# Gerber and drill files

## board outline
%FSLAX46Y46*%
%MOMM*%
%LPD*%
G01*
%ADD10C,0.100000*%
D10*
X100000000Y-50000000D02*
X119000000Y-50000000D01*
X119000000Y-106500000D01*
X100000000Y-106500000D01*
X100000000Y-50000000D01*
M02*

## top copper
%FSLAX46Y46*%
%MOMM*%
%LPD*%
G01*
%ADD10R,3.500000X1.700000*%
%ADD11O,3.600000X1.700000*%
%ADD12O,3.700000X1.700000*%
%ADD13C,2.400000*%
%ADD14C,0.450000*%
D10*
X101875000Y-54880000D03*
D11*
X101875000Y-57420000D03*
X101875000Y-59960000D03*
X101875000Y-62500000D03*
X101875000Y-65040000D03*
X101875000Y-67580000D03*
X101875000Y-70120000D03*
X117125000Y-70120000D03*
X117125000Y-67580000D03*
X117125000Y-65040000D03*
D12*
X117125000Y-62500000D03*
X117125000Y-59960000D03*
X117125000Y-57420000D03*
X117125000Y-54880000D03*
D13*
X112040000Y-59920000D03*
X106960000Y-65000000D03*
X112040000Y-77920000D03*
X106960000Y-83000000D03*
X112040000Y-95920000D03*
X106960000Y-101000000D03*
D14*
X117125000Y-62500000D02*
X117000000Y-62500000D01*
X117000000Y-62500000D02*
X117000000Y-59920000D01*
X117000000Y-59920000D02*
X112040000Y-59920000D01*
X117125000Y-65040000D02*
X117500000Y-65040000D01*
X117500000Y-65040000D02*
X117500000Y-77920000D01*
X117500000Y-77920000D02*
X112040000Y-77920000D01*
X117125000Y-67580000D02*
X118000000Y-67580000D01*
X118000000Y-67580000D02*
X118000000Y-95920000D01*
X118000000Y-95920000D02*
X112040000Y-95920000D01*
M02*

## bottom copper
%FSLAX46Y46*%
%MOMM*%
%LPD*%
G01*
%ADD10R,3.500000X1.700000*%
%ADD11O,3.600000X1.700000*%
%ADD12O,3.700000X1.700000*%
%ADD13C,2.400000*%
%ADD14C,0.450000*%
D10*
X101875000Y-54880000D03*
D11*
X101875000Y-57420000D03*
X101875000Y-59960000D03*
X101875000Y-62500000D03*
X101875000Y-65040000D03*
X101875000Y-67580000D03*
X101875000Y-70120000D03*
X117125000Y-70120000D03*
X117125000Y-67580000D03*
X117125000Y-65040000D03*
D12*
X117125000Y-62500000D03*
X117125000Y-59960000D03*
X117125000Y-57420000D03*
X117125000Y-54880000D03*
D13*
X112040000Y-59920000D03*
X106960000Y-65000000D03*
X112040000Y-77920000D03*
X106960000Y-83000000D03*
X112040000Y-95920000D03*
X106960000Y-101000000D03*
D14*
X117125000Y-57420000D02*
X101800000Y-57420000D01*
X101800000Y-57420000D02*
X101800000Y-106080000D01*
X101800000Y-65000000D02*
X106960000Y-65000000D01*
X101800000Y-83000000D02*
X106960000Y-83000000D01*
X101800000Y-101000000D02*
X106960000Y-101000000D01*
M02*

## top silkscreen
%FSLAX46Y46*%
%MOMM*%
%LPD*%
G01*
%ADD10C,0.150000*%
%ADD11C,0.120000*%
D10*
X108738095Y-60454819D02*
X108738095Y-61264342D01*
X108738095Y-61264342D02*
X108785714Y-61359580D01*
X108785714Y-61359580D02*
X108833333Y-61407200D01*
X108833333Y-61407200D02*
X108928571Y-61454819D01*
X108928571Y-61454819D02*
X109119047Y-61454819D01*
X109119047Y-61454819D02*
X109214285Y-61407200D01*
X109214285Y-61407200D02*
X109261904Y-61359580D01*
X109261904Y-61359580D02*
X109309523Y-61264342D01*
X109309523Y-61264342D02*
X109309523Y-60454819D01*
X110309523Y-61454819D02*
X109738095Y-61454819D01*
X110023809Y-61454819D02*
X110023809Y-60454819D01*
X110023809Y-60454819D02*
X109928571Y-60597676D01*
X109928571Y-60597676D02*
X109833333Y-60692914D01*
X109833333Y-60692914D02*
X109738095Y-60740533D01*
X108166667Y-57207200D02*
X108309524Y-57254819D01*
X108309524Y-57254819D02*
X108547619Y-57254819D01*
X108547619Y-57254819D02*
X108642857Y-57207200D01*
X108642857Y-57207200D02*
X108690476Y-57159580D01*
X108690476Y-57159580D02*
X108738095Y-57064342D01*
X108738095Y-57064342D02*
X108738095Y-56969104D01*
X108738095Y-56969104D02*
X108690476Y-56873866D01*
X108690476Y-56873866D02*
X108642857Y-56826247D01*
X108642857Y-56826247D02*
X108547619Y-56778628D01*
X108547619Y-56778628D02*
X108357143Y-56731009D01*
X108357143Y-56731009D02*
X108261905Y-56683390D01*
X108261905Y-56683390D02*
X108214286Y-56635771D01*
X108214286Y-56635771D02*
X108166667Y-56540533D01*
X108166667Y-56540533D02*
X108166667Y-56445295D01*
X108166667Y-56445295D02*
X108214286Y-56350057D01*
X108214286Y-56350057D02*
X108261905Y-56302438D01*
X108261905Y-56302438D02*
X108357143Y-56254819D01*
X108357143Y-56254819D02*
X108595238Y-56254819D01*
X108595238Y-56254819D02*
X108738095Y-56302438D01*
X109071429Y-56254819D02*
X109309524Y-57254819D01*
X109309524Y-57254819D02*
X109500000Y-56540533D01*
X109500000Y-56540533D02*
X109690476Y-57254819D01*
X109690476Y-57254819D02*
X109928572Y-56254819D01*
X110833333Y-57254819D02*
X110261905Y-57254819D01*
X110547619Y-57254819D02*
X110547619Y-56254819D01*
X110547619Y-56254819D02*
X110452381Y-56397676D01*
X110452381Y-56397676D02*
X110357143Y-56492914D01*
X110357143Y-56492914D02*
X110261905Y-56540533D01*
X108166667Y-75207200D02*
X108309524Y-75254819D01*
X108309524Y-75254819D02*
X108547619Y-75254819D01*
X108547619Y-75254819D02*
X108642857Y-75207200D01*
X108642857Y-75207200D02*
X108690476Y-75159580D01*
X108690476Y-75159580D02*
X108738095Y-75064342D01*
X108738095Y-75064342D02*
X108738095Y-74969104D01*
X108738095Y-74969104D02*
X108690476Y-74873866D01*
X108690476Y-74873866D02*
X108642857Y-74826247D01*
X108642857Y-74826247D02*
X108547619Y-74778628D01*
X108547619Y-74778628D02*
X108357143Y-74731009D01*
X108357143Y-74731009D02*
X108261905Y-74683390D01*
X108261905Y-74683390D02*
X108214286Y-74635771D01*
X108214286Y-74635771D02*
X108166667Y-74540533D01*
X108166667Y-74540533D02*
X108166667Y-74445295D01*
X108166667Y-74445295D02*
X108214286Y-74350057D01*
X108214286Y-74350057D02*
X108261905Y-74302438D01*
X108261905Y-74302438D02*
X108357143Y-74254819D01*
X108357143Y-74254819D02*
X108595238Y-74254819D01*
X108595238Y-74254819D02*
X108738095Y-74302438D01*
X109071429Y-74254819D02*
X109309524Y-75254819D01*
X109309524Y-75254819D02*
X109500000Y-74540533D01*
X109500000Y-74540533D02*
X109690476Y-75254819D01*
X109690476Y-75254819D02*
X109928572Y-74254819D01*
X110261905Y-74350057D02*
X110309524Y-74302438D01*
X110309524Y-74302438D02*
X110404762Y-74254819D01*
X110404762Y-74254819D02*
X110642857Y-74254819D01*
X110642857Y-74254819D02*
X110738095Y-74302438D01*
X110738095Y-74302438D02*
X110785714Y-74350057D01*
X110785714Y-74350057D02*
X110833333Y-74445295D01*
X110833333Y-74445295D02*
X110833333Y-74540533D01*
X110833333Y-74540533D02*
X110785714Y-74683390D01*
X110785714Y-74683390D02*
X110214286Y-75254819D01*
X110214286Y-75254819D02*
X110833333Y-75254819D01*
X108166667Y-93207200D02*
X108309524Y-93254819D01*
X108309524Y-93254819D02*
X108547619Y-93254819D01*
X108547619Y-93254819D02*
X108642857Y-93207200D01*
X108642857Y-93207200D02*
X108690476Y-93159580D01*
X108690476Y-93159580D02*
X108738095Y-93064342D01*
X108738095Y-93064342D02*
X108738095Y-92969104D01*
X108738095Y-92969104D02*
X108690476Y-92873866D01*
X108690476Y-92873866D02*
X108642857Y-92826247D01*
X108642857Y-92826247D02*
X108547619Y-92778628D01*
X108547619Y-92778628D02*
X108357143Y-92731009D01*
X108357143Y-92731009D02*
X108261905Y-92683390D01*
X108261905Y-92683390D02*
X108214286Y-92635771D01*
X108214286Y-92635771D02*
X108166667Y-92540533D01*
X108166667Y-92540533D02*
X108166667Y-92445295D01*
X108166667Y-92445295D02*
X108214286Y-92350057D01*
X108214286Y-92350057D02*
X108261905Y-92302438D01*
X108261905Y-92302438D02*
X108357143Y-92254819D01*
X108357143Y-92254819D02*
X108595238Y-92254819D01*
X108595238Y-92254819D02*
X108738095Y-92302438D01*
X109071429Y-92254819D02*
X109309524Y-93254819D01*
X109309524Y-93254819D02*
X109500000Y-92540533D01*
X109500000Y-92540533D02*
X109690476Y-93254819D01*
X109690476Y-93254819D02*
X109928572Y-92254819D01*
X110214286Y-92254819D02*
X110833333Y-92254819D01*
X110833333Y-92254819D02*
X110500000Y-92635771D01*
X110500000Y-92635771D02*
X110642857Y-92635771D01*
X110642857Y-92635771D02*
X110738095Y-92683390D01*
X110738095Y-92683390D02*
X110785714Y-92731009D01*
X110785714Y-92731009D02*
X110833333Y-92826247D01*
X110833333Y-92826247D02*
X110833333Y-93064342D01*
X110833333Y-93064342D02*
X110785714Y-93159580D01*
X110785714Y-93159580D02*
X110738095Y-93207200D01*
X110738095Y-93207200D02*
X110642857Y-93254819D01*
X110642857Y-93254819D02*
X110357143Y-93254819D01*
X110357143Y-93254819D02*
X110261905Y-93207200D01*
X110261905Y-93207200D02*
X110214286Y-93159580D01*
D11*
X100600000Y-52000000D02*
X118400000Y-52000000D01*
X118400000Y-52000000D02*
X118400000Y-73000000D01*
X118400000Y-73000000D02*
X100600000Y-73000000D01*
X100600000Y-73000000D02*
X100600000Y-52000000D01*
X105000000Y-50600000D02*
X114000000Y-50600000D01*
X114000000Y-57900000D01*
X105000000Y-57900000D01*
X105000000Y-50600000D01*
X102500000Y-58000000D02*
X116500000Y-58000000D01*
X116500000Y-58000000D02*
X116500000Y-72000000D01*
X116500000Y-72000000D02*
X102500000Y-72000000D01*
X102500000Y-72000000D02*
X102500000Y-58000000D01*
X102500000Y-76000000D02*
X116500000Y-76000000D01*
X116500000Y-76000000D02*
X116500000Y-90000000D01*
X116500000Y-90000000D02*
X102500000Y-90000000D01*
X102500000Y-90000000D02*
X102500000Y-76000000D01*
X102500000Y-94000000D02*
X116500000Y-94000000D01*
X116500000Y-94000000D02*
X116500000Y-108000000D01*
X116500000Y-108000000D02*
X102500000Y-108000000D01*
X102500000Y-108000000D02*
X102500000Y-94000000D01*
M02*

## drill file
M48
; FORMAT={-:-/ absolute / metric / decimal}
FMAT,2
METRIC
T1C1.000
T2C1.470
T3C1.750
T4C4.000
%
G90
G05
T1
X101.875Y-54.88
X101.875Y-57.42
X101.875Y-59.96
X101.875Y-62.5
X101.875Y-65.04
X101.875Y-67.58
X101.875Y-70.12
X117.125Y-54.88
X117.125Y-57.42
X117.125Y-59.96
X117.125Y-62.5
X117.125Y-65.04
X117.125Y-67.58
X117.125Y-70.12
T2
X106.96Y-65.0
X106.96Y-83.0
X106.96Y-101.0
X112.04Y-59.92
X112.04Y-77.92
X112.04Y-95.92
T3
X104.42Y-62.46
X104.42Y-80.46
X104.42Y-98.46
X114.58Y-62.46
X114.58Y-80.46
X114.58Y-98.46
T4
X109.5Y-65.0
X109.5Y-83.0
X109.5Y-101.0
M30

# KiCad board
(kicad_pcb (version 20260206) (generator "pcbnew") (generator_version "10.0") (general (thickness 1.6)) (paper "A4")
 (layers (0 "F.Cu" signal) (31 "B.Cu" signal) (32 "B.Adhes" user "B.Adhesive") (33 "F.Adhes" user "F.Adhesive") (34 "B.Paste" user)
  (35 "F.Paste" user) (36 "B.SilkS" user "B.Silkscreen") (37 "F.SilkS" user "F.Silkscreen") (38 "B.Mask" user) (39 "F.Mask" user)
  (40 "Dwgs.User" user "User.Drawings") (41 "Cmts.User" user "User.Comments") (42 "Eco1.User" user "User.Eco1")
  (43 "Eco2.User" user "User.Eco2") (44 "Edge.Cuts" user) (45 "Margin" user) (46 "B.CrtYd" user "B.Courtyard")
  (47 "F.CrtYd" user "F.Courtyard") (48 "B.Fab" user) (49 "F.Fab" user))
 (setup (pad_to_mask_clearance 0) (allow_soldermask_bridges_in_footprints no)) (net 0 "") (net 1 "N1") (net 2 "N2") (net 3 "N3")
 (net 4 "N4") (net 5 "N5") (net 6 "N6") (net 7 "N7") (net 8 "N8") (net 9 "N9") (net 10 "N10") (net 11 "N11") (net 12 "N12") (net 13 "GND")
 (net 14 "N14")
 (gr_rect (start 100.000 50.000) (end 119.000 106.500) (stroke (width 0.1) (type solid)) (fill no) (layer "Edge.Cuts"))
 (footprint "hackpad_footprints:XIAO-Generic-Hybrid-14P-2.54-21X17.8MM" (layer "F.Cu") (at 109.500 62.500 0)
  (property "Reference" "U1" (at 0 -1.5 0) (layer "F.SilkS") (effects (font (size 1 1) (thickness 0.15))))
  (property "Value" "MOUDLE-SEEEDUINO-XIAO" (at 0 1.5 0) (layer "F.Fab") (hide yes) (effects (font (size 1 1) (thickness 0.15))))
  (fp_line (start -8.9 -10.5) (end 8.9 -10.5) (stroke (width 0.12) (type solid)) (layer "F.SilkS"))
  (fp_line (start 8.9 -10.5) (end 8.9 10.5) (stroke (width 0.12) (type solid)) (layer "F.SilkS"))
  (fp_line (start 8.9 10.5) (end -8.9 10.5) (stroke (width 0.12) (type solid)) (layer "F.SilkS"))
  (fp_line (start -8.9 10.5) (end -8.9 -10.5) (stroke (width 0.12) (type solid)) (layer "F.SilkS"))
  (fp_rect (start -4.5 -11.9) (end 4.5 -4.6) (stroke (width 0.12) (type solid)) (fill no) (layer "F.SilkS"))
  (pad "1" thru_hole rect (at -7.625 -7.620) (size 3.5 1.7) (drill 1) (layers "*.Cu" "*.Mask") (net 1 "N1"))
  (pad "2" thru_hole oval (at -7.625 -5.080) (size 3.6 1.7) (drill 1) (layers "*.Cu" "*.Mask") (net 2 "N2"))
  (pad "3" thru_hole oval (at -7.625 -2.540) (size 3.6 1.7) (drill 1) (layers "*.Cu" "*.Mask") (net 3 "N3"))
  (pad "4" thru_hole oval (at -7.625 0.000) (size 3.6 1.7) (drill 1) (layers "*.Cu" "*.Mask") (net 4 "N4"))
  (pad "5" thru_hole oval (at -7.625 2.540) (size 3.6 1.7) (drill 1) (layers "*.Cu" "*.Mask") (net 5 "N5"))
  (pad "6" thru_hole oval (at -7.625 5.080) (size 3.6 1.7) (drill 1) (layers "*.Cu" "*.Mask") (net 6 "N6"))
  (pad "7" thru_hole oval (at -7.625 7.620) (size 3.6 1.7) (drill 1) (layers "*.Cu" "*.Mask") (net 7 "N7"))
  (pad "8" thru_hole oval (at 7.625 7.620) (size 3.6 1.7) (drill 1) (layers "*.Cu" "*.Mask") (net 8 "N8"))
  (pad "9" thru_hole oval (at 7.625 5.080) (size 3.6 1.7) (drill 1) (layers "*.Cu" "*.Mask") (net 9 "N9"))
  (pad "10" thru_hole oval (at 7.625 2.540) (size 3.6 1.7) (drill 1) (layers "*.Cu" "*.Mask") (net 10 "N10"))
  (pad "11" thru_hole oval (at 7.625 0.000) (size 3.7 1.7) (drill 1) (layers "*.Cu" "*.Mask") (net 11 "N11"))
  (pad "12" thru_hole oval (at 7.625 -2.540) (size 3.7 1.7) (drill 1) (layers "*.Cu" "*.Mask") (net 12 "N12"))
  (pad "13" thru_hole oval (at 7.625 -5.080) (size 3.7 1.7) (drill 1) (layers "*.Cu" "*.Mask") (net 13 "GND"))
  (pad "14" thru_hole oval (at 7.625 -7.620) (size 3.7 1.7) (drill 1) (layers "*.Cu" "*.Mask") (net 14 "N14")))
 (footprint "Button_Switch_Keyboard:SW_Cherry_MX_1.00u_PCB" (layer "F.Cu") (at 109.500 65.000 0)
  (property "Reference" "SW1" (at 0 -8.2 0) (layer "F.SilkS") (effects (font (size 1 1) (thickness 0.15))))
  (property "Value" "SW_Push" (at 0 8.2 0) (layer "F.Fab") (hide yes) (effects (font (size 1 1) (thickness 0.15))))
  (fp_line (start -7 -7) (end 7 -7) (stroke (width 0.12) (type solid)) (layer "F.SilkS"))
  (fp_line (start 7 -7) (end 7 7) (stroke (width 0.12) (type solid)) (layer "F.SilkS"))
  (fp_line (start 7 7) (end -7 7) (stroke (width 0.12) (type solid)) (layer "F.SilkS"))
  (fp_line (start -7 7) (end -7 -7) (stroke (width 0.12) (type solid)) (layer "F.SilkS"))
  (pad "" np_thru_hole circle (at -5.08 -2.54) (size 1.75 1.75) (drill 1.75) (layers "*.Cu" "*.Mask"))
  (pad "" np_thru_hole circle (at 5.08 -2.54) (size 1.75 1.75) (drill 1.75) (layers "*.Cu" "*.Mask"))
  (pad "" np_thru_hole circle (at 0 0) (size 4 4) (drill 4) (layers "*.Cu" "*.Mask"))
  (pad "1" thru_hole circle (at 2.54 -5.08) (size 2.4 2.4) (drill 1.47) (layers "*.Cu" "*.Mask") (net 11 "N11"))
  (pad "2" thru_hole circle (at -2.54 0) (size 2.4 2.4) (drill 1.47) (layers "*.Cu" "*.Mask") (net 13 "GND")))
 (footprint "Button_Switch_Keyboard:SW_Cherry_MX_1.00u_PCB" (layer "F.Cu") (at 109.500 83.000 0)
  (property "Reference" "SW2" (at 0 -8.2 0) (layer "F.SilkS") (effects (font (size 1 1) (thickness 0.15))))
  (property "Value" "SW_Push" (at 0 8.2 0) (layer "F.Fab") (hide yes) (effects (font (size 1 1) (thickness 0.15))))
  (fp_line (start -7 -7) (end 7 -7) (stroke (width 0.12) (type solid)) (layer "F.SilkS"))
  (fp_line (start 7 -7) (end 7 7) (stroke (width 0.12) (type solid)) (layer "F.SilkS"))
  (fp_line (start 7 7) (end -7 7) (stroke (width 0.12) (type solid)) (layer "F.SilkS"))
  (fp_line (start -7 7) (end -7 -7) (stroke (width 0.12) (type solid)) (layer "F.SilkS"))
  (pad "" np_thru_hole circle (at -5.08 -2.54) (size 1.75 1.75) (drill 1.75) (layers "*.Cu" "*.Mask"))
  (pad "" np_thru_hole circle (at 5.08 -2.54) (size 1.75 1.75) (drill 1.75) (layers "*.Cu" "*.Mask"))
  (pad "" np_thru_hole circle (at 0 0) (size 4 4) (drill 4) (layers "*.Cu" "*.Mask"))
  (pad "1" thru_hole circle (at 2.54 -5.08) (size 2.4 2.4) (drill 1.47) (layers "*.Cu" "*.Mask") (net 10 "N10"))
  (pad "2" thru_hole circle (at -2.54 0) (size 2.4 2.4) (drill 1.47) (layers "*.Cu" "*.Mask") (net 13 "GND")))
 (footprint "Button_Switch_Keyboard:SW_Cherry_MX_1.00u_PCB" (layer "F.Cu") (at 109.500 101.000 0)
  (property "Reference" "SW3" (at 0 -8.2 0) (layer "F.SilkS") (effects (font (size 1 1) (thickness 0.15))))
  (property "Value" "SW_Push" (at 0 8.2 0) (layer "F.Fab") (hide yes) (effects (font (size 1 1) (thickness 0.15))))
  (fp_line (start -7 -7) (end 7 -7) (stroke (width 0.12) (type solid)) (layer "F.SilkS"))
  (fp_line (start 7 -7) (end 7 7) (stroke (width 0.12) (type solid)) (layer "F.SilkS"))
  (fp_line (start 7 7) (end -7 7) (stroke (width 0.12) (type solid)) (layer "F.SilkS"))
  (fp_line (start -7 7) (end -7 -7) (stroke (width 0.12) (type solid)) (layer "F.SilkS"))
  (pad "" np_thru_hole circle (at -5.08 -2.54) (size 1.75 1.75) (drill 1.75) (layers "*.Cu" "*.Mask"))
  (pad "" np_thru_hole circle (at 5.08 -2.54) (size 1.75 1.75) (drill 1.75) (layers "*.Cu" "*.Mask"))
  (pad "" np_thru_hole circle (at 0 0) (size 4 4) (drill 4) (layers "*.Cu" "*.Mask"))
  (pad "1" thru_hole circle (at 2.54 -5.08) (size 2.4 2.4) (drill 1.47) (layers "*.Cu" "*.Mask") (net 9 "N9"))
  (pad "2" thru_hole circle (at -2.54 0) (size 2.4 2.4) (drill 1.47) (layers "*.Cu" "*.Mask") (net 13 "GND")))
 (segment (start 117.125 62.500) (end 117.000 62.500) (width 0.45) (layer "F.Cu") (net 11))
 (segment (start 117.000 62.500) (end 117.000 59.920) (width 0.45) (layer "F.Cu") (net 11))
 (segment (start 117.000 59.920) (end 112.040 59.920) (width 0.45) (layer "F.Cu") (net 11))
 (segment (start 117.125 65.040) (end 117.500 65.040) (width 0.45) (layer "F.Cu") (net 10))
 (segment (start 117.500 65.040) (end 117.500 77.920) (width 0.45) (layer "F.Cu") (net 10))
 (segment (start 117.500 77.920) (end 112.040 77.920) (width 0.45) (layer "F.Cu") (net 10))
 (segment (start 117.125 67.580) (end 118.000 67.580) (width 0.45) (layer "F.Cu") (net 9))
 (segment (start 118.000 67.580) (end 118.000 95.920) (width 0.45) (layer "F.Cu") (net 9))
 (segment (start 118.000 95.920) (end 112.040 95.920) (width 0.45) (layer "F.Cu") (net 9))
 (segment (start 117.125 57.420) (end 101.800 57.420) (width 0.45) (layer "B.Cu") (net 13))
 (segment (start 101.800 57.420) (end 101.800 106.080) (width 0.45) (layer "B.Cu") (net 13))
 (segment (start 101.800 65.000) (end 106.960 65.000) (width 0.45) (layer "B.Cu") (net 13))
 (segment (start 101.800 83.000) (end 106.960 83.000) (width 0.45) (layer "B.Cu") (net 13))
 (segment (start 101.800 101.000) (end 106.960 101.000) (width 0.45) (layer "B.Cu") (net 13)))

